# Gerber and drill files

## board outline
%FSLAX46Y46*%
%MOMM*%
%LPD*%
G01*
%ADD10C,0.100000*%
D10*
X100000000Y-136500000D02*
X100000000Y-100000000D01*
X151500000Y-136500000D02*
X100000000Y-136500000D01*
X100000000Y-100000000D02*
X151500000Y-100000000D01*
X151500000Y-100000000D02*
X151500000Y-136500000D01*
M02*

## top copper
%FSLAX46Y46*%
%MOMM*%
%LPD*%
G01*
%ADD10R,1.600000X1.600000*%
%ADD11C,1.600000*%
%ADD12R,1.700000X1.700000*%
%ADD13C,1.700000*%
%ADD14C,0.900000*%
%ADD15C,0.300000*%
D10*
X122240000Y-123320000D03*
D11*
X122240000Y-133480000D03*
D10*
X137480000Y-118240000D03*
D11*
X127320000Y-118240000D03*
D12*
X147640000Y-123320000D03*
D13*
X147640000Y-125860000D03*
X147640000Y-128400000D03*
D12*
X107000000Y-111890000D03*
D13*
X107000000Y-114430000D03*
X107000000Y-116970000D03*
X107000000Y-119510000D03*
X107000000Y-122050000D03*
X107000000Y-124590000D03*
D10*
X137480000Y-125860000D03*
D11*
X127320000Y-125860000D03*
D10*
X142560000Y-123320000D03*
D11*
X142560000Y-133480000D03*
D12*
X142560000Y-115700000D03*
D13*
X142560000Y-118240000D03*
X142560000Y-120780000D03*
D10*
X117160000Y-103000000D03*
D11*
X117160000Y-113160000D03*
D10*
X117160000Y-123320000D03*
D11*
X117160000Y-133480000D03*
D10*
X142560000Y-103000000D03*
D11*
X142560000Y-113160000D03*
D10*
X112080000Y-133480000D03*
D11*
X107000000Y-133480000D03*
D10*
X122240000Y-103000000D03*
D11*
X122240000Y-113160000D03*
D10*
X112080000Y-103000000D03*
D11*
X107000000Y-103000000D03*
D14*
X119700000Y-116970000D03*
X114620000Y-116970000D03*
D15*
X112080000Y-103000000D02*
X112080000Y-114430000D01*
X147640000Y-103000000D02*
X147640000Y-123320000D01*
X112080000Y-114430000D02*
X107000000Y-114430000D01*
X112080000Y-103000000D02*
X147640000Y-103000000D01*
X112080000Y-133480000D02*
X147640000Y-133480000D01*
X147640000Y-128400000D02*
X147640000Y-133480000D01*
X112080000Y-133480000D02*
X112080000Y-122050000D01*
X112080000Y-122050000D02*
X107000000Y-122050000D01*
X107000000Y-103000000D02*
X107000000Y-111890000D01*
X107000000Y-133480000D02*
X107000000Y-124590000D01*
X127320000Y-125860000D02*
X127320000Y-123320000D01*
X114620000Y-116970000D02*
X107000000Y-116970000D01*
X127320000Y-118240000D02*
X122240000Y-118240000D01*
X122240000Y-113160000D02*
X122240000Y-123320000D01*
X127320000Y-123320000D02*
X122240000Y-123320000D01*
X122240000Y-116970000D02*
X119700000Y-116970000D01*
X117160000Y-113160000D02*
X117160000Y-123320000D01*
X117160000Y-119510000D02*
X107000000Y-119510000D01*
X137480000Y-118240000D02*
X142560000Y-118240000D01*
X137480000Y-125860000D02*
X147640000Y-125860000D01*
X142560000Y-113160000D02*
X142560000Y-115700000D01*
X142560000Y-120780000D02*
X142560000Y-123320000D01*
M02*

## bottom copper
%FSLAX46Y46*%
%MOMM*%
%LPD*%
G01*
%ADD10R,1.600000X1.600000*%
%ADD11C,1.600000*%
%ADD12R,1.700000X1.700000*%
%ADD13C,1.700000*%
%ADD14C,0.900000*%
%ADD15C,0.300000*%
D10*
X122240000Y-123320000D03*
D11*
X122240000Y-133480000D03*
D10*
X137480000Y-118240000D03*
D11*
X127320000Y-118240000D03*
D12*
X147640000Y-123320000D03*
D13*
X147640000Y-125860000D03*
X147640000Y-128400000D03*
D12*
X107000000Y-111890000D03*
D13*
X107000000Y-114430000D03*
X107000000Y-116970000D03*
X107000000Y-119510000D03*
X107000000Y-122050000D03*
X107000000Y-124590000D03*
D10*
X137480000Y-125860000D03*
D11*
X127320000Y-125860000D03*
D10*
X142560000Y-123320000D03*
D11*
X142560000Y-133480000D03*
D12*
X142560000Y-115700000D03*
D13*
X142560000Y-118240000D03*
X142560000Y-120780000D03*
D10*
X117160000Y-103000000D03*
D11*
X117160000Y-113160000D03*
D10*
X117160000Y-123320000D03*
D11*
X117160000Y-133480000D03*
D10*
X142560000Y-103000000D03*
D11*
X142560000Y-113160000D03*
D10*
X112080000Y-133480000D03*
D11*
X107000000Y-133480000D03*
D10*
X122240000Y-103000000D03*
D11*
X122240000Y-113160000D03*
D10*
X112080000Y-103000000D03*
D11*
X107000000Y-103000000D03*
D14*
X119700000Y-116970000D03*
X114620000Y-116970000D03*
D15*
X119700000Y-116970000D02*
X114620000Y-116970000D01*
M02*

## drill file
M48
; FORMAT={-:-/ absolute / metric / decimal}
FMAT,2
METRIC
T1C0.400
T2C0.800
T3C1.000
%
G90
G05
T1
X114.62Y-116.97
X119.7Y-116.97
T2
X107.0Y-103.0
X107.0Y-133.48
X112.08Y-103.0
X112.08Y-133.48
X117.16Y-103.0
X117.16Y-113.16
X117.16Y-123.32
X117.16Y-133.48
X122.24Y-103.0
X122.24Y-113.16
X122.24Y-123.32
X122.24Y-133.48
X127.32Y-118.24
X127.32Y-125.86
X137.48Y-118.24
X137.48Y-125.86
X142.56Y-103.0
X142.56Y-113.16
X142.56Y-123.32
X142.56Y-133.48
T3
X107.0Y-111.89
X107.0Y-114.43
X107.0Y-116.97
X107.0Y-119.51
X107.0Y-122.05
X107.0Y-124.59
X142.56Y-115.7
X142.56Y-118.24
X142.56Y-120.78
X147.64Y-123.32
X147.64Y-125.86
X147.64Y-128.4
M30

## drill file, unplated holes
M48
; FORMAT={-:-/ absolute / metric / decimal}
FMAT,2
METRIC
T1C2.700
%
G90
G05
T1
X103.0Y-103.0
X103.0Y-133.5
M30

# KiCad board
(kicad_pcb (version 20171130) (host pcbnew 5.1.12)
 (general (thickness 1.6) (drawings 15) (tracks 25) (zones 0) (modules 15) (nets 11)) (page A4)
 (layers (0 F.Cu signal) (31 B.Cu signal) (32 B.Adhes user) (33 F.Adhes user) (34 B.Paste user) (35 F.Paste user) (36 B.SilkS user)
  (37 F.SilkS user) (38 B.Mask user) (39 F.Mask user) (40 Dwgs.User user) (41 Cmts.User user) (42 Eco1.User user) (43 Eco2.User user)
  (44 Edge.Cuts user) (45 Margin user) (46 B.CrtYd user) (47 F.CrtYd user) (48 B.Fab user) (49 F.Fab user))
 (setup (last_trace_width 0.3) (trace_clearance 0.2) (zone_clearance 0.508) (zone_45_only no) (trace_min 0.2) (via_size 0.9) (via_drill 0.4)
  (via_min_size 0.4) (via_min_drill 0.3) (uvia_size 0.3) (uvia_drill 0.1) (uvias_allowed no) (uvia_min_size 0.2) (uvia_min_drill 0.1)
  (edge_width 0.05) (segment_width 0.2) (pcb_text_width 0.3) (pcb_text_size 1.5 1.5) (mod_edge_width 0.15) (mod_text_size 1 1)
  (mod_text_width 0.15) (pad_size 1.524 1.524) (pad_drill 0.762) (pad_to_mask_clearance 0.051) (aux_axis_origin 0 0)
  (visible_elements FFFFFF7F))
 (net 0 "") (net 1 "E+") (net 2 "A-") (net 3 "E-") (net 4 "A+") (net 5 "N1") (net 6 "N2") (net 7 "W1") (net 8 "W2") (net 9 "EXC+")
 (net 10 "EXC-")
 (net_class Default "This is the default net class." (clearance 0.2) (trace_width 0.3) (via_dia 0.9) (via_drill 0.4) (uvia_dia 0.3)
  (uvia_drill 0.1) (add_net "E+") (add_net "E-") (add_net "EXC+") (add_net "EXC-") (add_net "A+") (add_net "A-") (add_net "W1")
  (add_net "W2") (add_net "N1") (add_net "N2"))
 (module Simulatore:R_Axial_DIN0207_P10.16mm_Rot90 (layer F.Cu) (at 117.16 103)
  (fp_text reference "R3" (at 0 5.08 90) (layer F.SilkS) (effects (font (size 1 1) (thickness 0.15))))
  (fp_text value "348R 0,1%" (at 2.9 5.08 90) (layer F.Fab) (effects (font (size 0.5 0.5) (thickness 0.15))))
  (pad 1 thru_hole rect (at 0 0) (size 1.6 1.6) (drill 0.8) (layers *.Cu *.Mask) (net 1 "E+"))
  (pad 2 thru_hole circle (at 0 10.16) (size 1.6 1.6) (drill 0.8) (layers *.Cu *.Mask) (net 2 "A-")))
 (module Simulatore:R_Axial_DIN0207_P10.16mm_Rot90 (layer F.Cu) (at 117.16 123.32)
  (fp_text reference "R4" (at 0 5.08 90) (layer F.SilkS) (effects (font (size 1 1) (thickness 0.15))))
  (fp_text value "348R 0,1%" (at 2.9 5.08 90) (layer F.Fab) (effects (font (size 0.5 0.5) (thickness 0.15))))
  (pad 1 thru_hole rect (at 0 0) (size 1.6 1.6) (drill 0.8) (layers *.Cu *.Mask) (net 2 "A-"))
  (pad 2 thru_hole circle (at 0 10.16) (size 1.6 1.6) (drill 0.8) (layers *.Cu *.Mask) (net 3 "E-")))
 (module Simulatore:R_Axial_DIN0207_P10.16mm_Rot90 (layer F.Cu) (at 122.24 103)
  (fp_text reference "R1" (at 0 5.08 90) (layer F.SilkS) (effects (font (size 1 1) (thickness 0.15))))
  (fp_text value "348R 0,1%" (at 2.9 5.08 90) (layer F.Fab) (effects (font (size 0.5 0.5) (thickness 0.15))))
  (pad 1 thru_hole rect (at 0 0) (size 1.6 1.6) (drill 0.8) (layers *.Cu *.Mask) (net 1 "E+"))
  (pad 2 thru_hole circle (at 0 10.16) (size 1.6 1.6) (drill 0.8) (layers *.Cu *.Mask) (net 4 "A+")))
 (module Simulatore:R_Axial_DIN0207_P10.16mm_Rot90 (layer F.Cu) (at 122.24 123.32)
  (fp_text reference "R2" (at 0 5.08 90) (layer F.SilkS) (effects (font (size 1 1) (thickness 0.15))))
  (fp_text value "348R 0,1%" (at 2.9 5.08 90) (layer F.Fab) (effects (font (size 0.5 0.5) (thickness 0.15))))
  (pad 1 thru_hole rect (at 0 0) (size 1.6 1.6) (drill 0.8) (layers *.Cu *.Mask) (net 4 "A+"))
  (pad 2 thru_hole circle (at 0 10.16) (size 1.6 1.6) (drill 0.8) (layers *.Cu *.Mask) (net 3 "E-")))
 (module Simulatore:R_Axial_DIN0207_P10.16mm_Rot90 (layer F.Cu) (at 142.56 103)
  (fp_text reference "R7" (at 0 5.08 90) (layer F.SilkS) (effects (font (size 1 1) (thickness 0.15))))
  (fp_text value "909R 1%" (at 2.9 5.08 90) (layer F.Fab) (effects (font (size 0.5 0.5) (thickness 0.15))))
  (pad 1 thru_hole rect (at 0 0) (size 1.6 1.6) (drill 0.8) (layers *.Cu *.Mask) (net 1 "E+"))
  (pad 2 thru_hole circle (at 0 10.16) (size 1.6 1.6) (drill 0.8) (layers *.Cu *.Mask) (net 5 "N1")))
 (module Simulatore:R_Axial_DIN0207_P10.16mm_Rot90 (layer F.Cu) (at 142.56 123.32)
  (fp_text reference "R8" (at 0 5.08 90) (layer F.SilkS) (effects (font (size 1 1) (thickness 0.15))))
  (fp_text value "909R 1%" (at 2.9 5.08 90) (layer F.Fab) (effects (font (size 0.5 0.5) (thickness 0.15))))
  (pad 1 thru_hole rect (at 0 0) (size 1.6 1.6) (drill 0.8) (layers *.Cu *.Mask) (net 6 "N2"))
  (pad 2 thru_hole circle (at 0 10.16) (size 1.6 1.6) (drill 0.8) (layers *.Cu *.Mask) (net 3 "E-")))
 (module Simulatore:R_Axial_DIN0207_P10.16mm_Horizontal (layer F.Cu) (at 132.4 118.24)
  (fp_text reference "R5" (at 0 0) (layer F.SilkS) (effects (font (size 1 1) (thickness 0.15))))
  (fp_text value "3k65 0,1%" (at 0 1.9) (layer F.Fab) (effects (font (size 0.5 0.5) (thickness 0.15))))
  (pad 1 thru_hole rect (at 5.08 0) (size 1.6 1.6) (drill 0.8) (layers *.Cu *.Mask) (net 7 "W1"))
  (pad 2 thru_hole circle (at -5.08 0) (size 1.6 1.6) (drill 0.8) (layers *.Cu *.Mask) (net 4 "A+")))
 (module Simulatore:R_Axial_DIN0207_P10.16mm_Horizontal (layer F.Cu) (at 132.4 125.86)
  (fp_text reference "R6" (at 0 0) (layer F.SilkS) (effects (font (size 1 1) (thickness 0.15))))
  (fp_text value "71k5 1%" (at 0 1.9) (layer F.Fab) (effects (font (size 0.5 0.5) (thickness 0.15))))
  (pad 1 thru_hole rect (at 5.08 0) (size 1.6 1.6) (drill 0.8) (layers *.Cu *.Mask) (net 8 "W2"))
  (pad 2 thru_hole circle (at -5.08 0) (size 1.6 1.6) (drill 0.8) (layers *.Cu *.Mask) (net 4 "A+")))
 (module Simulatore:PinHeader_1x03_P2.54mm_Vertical (layer F.Cu) (at 142.56 115.7)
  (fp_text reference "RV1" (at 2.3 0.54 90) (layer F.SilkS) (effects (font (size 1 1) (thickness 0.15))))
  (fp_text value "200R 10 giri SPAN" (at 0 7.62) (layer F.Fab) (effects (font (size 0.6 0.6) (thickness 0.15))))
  (pad 1 thru_hole rect (at 0 0) (size 1.7 1.7) (drill 1) (layers *.Cu *.Mask) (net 5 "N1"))
  (pad 2 thru_hole circle (at 0 2.54) (size 1.7 1.7) (drill 1) (layers *.Cu *.Mask) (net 7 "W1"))
  (pad 3 thru_hole circle (at 0 5.08) (size 1.7 1.7) (drill 1) (layers *.Cu *.Mask) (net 6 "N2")))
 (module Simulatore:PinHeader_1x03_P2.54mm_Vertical (layer F.Cu) (at 147.64 123.32)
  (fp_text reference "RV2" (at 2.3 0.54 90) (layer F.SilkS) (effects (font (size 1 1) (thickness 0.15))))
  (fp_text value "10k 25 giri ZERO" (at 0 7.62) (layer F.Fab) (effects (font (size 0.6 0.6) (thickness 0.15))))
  (pad 1 thru_hole rect (at 0 0) (size 1.7 1.7) (drill 1) (layers *.Cu *.Mask) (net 1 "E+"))
  (pad 2 thru_hole circle (at 0 2.54) (size 1.7 1.7) (drill 1) (layers *.Cu *.Mask) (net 8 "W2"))
  (pad 3 thru_hole circle (at 0 5.08) (size 1.7 1.7) (drill 1) (layers *.Cu *.Mask) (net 3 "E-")))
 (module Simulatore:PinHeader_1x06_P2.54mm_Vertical (layer F.Cu) (at 107 111.89)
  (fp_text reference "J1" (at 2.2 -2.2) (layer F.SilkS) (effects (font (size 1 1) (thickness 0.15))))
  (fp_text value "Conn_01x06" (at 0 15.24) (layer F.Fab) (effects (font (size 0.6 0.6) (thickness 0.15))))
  (pad 1 thru_hole rect (at 0 0) (size 1.7 1.7) (drill 1) (layers *.Cu *.Mask) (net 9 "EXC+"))
  (pad 2 thru_hole circle (at 0 2.54) (size 1.7 1.7) (drill 1) (layers *.Cu *.Mask) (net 1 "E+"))
  (pad 3 thru_hole circle (at 0 5.08) (size 1.7 1.7) (drill 1) (layers *.Cu *.Mask) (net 4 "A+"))
  (pad 4 thru_hole circle (at 0 7.62) (size 1.7 1.7) (drill 1) (layers *.Cu *.Mask) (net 2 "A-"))
  (pad 5 thru_hole circle (at 0 10.16) (size 1.7 1.7) (drill 1) (layers *.Cu *.Mask) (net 3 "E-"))
  (pad 6 thru_hole circle (at 0 12.7) (size 1.7 1.7) (drill 1) (layers *.Cu *.Mask) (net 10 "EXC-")))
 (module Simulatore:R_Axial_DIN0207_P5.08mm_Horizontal (layer F.Cu) (at 112.08 103)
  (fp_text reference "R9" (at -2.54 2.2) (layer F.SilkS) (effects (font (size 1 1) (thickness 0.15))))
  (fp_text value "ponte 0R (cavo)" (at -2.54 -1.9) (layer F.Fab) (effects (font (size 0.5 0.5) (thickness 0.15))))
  (pad 1 thru_hole rect (at 0 0) (size 1.6 1.6) (drill 0.8) (layers *.Cu *.Mask) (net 1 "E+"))
  (pad 2 thru_hole circle (at -5.08 0) (size 1.6 1.6) (drill 0.8) (layers *.Cu *.Mask) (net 9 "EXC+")))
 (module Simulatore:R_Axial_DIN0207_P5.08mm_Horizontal (layer F.Cu) (at 112.08 133.48)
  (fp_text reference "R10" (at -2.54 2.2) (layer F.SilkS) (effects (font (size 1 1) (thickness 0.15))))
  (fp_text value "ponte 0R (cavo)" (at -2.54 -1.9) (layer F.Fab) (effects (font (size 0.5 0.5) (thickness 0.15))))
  (pad 1 thru_hole rect (at 0 0) (size 1.6 1.6) (drill 0.8) (layers *.Cu *.Mask) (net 3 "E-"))
  (pad 2 thru_hole circle (at -5.08 0) (size 1.6 1.6) (drill 0.8) (layers *.Cu *.Mask) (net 10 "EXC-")))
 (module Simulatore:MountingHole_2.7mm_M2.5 (layer F.Cu) (at 103 103)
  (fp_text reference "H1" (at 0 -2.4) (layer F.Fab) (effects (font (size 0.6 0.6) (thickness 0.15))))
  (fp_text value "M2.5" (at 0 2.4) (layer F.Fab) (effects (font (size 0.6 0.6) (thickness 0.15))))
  (pad "" np_thru_hole circle (at 0 0) (size 2.7 2.7) (drill 2.7) (layers *.Cu *.Mask)))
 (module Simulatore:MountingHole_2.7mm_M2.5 (layer F.Cu) (at 103 133.5)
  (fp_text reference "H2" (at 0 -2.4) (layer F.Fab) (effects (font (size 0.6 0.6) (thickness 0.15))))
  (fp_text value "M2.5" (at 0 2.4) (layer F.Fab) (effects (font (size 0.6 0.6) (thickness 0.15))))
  (pad "" np_thru_hole circle (at 0 0) (size 2.7 2.7) (drill 2.7) (layers *.Cu *.Mask)))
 (gr_line (start 100 100) (end 151.5 100) (layer Edge.Cuts) (width 0.05))
 (gr_line (start 151.5 100) (end 151.5 136.5) (layer Edge.Cuts) (width 0.05))
 (gr_line (start 151.5 136.5) (end 100 136.5) (layer Edge.Cuts) (width 0.05))
 (gr_line (start 100 136.5) (end 100 100) (layer Edge.Cuts) (width 0.05))
 (segment (start 112.08 103) (end 147.64 103) (width 0.3) (layer F.Cu) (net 1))
 (segment (start 112.08 133.48) (end 147.64 133.48) (width 0.3) (layer F.Cu) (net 3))
 (segment (start 107 103) (end 107 111.89) (width 0.3) (layer F.Cu) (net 9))
 (segment (start 107 133.48) (end 107 124.59) (width 0.3) (layer F.Cu) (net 10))
 (segment (start 112.08 103) (end 112.08 114.43) (width 0.3) (layer F.Cu) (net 1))
 (segment (start 112.08 114.43) (end 107 114.43) (width 0.3) (layer F.Cu) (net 1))
 (segment (start 112.08 133.48) (end 112.08 122.05) (width 0.3) (layer F.Cu) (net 3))
 (segment (start 112.08 122.05) (end 107 122.05) (width 0.3) (layer F.Cu) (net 3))
 (segment (start 117.16 113.16) (end 117.16 123.32) (width 0.3) (layer F.Cu) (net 2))
 (segment (start 117.16 119.51) (end 107 119.51) (width 0.3) (layer F.Cu) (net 2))
 (segment (start 122.24 113.16) (end 122.24 123.32) (width 0.3) (layer F.Cu) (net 4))
 (segment (start 122.24 116.97) (end 119.7 116.97) (width 0.3) (layer F.Cu) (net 4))
 (segment (start 119.7 116.97) (end 114.62 116.97) (width 0.3) (layer B.Cu) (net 4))
 (segment (start 114.62 116.97) (end 107 116.97) (width 0.3) (layer F.Cu) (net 4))
 (segment (start 127.32 118.24) (end 122.24 118.24) (width 0.3) (layer F.Cu) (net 4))
 (segment (start 127.32 125.86) (end 127.32 123.32) (width 0.3) (layer F.Cu) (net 4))
 (segment (start 127.32 123.32) (end 122.24 123.32) (width 0.3) (layer F.Cu) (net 4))
 (segment (start 137.48 118.24) (end 142.56 118.24) (width 0.3) (layer F.Cu) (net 7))
 (segment (start 137.48 125.86) (end 147.64 125.86) (width 0.3) (layer F.Cu) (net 8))
 (segment (start 142.56 113.16) (end 142.56 115.7) (width 0.3) (layer F.Cu) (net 5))
 (segment (start 142.56 120.78) (end 142.56 123.32) (width 0.3) (layer F.Cu) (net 6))
 (segment (start 147.64 103) (end 147.64 123.32) (width 0.3) (layer F.Cu) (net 1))
 (segment (start 147.64 128.4) (end 147.64 133.48) (width 0.3) (layer F.Cu) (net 3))
 (via (at 119.7 116.97) (size 0.9) (drill 0.4) (layers F.Cu B.Cu) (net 4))
 (via (at 114.62 116.97) (size 0.9) (drill 0.4) (layers F.Cu B.Cu) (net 4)))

